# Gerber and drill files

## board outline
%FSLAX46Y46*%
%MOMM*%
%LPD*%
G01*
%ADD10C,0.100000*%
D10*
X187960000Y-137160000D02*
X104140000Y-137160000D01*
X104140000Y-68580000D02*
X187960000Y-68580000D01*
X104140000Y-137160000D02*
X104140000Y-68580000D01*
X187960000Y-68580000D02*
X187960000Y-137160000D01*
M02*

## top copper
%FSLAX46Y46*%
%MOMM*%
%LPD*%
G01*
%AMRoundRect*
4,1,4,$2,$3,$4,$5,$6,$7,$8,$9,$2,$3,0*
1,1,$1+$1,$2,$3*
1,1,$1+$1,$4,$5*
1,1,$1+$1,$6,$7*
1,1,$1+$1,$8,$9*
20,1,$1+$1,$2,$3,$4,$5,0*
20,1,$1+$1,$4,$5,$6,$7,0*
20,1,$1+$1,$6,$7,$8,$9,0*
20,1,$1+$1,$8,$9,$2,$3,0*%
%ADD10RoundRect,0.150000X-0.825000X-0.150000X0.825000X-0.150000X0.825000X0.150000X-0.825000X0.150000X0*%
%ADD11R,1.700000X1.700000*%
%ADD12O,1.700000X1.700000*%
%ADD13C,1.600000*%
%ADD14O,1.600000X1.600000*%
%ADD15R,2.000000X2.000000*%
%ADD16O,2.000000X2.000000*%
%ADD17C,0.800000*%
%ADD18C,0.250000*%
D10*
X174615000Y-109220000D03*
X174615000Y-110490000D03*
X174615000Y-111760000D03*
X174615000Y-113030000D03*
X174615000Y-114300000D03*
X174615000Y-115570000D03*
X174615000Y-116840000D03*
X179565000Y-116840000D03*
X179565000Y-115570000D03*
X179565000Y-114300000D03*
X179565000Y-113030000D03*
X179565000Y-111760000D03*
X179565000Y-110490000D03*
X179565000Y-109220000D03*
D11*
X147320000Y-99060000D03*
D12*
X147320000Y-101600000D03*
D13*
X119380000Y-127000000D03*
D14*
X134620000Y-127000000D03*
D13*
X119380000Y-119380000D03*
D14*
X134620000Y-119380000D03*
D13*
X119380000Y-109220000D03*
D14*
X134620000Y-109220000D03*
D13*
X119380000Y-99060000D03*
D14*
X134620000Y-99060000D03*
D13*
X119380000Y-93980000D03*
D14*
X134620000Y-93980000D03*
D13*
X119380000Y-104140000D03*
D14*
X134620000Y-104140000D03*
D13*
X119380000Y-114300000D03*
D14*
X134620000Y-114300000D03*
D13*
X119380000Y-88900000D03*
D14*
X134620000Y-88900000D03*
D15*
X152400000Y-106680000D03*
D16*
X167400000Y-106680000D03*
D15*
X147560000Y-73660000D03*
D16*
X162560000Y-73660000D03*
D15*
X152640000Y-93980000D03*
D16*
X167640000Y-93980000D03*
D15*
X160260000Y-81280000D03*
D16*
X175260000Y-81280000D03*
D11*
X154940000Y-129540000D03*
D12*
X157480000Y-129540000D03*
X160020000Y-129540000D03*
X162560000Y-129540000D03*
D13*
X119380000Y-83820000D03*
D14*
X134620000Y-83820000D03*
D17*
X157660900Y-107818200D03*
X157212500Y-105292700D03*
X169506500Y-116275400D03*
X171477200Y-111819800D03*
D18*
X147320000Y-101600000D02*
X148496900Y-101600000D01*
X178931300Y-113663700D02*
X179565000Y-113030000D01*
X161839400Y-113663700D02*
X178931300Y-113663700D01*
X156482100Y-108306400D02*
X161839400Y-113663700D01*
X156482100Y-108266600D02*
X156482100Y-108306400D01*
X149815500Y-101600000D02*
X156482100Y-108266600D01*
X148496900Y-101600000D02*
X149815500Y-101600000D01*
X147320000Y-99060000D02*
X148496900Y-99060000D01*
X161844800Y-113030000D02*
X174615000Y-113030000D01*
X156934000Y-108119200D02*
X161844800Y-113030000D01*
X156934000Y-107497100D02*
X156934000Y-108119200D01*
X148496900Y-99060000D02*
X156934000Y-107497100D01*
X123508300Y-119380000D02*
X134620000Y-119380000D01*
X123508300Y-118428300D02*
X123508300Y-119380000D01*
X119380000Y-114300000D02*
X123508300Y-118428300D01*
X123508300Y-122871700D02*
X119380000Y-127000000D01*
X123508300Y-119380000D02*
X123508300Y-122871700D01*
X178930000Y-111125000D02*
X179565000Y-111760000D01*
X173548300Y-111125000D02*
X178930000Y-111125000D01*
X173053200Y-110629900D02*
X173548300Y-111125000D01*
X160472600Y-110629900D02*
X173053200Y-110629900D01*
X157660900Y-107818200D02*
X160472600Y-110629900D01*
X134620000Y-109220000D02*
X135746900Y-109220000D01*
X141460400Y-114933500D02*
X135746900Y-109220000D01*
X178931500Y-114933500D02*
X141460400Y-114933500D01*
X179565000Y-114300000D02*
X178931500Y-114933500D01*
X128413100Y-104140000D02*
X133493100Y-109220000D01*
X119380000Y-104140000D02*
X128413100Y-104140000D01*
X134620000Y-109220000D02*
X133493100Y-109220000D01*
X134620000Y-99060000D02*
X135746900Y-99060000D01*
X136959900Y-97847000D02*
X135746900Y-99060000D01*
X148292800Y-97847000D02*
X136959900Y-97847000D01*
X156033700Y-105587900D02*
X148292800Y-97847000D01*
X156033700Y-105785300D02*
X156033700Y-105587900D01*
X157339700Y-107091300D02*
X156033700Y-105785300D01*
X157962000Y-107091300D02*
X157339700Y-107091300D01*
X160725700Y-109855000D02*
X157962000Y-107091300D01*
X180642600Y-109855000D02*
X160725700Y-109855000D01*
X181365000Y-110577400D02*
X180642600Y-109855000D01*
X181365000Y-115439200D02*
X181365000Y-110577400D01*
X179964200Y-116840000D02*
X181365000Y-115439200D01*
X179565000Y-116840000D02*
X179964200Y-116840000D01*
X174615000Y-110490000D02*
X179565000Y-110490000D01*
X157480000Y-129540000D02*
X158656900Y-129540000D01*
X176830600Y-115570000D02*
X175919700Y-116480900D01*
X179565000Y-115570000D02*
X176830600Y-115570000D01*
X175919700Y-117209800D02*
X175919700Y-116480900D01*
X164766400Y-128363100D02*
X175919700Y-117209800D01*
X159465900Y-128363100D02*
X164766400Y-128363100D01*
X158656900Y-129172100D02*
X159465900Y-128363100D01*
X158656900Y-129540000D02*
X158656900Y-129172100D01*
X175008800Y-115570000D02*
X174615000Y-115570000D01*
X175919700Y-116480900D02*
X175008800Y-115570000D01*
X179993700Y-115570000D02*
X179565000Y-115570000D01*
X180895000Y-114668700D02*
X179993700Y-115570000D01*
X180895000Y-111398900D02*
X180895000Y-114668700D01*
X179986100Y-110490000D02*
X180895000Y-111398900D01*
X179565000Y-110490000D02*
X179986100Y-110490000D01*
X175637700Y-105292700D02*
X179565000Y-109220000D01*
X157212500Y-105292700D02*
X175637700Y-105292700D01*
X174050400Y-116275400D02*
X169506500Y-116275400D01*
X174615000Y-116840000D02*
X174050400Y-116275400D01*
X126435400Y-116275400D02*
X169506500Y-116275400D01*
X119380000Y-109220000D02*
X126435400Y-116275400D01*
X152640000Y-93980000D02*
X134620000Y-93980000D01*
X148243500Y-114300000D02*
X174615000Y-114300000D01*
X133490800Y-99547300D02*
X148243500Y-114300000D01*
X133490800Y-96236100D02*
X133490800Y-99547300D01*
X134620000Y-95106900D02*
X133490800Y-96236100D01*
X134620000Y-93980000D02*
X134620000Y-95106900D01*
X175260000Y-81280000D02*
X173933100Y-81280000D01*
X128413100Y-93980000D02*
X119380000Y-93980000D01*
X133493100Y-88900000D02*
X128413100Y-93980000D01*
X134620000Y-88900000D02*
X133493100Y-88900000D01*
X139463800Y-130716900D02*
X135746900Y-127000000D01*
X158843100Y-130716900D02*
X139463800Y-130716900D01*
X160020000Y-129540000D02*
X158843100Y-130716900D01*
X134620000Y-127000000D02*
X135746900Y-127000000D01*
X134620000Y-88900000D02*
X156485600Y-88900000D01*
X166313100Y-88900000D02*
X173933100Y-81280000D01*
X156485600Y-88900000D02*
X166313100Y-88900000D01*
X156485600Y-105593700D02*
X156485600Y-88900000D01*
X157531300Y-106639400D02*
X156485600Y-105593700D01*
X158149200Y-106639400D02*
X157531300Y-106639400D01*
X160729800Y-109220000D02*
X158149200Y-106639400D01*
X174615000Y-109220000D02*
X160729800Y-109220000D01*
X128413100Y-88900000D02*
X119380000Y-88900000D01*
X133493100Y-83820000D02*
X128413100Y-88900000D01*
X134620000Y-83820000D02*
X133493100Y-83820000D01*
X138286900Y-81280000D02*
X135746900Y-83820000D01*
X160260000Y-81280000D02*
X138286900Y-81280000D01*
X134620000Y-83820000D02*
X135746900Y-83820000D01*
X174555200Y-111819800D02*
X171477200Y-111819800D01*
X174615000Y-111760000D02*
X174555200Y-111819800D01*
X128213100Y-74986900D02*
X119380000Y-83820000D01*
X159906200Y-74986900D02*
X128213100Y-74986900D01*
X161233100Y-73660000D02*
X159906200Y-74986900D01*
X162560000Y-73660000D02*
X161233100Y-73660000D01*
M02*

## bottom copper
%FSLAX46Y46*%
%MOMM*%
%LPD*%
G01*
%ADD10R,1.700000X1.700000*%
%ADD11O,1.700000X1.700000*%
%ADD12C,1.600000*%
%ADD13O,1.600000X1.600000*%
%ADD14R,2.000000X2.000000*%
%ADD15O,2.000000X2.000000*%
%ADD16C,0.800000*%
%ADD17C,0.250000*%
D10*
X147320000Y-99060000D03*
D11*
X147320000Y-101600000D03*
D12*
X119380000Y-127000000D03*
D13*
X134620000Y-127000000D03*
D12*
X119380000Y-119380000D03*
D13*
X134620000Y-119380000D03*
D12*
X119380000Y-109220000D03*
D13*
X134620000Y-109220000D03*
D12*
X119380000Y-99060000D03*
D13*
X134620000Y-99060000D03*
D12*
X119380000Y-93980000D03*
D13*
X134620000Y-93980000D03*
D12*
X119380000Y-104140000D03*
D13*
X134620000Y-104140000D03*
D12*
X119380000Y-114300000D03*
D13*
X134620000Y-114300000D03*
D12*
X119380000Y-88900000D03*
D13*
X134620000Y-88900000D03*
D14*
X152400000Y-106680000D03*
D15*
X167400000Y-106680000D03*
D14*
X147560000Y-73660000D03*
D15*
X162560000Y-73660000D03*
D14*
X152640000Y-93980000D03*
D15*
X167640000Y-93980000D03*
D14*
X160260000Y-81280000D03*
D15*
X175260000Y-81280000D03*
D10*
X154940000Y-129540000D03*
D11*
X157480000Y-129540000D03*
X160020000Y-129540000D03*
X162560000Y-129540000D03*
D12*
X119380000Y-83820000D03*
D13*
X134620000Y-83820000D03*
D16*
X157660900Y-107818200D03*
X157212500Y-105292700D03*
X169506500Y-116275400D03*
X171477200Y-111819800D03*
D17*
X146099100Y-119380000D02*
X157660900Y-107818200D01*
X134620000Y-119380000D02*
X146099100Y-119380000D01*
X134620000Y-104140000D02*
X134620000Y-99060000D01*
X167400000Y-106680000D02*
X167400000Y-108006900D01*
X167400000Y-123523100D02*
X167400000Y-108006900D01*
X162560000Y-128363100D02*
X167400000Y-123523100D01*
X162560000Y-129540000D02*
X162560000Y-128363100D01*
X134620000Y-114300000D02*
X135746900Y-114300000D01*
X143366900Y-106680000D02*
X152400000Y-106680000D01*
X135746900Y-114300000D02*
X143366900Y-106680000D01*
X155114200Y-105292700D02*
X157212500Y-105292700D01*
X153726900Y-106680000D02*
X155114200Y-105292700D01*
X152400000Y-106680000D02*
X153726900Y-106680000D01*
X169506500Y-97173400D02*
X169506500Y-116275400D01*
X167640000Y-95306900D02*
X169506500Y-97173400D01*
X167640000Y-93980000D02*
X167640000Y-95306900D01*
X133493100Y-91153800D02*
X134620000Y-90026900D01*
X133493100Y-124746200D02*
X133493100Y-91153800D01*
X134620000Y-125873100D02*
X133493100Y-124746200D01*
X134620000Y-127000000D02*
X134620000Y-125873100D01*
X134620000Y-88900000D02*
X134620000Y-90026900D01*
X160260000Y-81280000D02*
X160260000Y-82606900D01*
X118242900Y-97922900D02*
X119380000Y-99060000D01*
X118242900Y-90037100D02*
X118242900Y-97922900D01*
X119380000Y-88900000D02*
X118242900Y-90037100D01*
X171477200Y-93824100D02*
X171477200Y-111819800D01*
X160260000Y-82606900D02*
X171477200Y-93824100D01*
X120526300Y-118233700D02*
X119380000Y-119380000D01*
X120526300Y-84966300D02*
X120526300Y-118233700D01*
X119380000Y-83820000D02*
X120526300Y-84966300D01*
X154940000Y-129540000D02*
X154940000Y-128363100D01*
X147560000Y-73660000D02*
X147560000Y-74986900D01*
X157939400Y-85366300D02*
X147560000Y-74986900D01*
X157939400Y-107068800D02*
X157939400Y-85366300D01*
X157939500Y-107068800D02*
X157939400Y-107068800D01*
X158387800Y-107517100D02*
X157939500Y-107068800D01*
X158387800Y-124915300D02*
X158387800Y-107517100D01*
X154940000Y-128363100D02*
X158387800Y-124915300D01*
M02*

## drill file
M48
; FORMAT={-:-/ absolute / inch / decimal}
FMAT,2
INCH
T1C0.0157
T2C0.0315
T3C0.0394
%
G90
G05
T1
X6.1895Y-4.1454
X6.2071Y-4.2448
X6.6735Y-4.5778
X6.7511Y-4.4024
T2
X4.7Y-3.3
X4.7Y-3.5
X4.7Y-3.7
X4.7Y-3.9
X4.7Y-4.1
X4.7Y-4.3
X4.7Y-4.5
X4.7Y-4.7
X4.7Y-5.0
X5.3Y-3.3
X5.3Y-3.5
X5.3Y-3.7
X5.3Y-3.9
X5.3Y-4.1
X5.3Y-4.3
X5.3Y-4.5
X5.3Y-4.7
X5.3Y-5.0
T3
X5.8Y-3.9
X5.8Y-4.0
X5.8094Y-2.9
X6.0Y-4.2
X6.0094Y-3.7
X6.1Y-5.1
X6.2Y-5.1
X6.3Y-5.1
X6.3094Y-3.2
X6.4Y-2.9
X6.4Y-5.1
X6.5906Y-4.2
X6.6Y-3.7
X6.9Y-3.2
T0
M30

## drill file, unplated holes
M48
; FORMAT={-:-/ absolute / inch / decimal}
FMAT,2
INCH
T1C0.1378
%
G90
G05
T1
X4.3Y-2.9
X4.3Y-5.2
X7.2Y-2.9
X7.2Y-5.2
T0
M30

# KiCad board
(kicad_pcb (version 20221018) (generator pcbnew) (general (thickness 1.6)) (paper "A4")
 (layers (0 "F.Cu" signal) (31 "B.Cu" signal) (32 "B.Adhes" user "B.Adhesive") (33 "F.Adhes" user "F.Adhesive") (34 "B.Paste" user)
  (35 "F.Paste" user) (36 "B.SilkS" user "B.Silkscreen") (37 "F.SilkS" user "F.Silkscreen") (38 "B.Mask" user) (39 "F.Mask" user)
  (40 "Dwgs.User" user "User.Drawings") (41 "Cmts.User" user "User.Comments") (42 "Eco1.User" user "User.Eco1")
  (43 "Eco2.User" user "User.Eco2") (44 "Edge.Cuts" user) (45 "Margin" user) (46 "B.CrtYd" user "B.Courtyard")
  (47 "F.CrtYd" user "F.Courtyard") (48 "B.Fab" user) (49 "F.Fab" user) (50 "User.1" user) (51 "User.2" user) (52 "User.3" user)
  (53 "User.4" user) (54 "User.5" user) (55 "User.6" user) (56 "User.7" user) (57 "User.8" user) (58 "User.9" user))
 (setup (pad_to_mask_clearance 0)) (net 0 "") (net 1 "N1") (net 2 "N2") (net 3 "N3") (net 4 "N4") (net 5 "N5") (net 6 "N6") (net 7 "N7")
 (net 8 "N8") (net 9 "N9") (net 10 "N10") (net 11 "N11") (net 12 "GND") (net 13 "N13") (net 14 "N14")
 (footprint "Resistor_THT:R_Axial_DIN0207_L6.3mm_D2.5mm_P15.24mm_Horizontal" (layer "F.Cu") (at 119.38 127)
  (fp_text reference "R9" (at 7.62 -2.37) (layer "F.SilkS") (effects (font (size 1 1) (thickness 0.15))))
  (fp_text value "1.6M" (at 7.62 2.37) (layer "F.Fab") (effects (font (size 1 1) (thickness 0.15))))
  (pad "1" thru_hole circle (at 0 0) (size 1.6 1.6) (drill 0.8) (layers "*.Cu" "*.Mask") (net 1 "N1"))
  (pad "2" thru_hole oval (at 15.24 0) (size 1.6 1.6) (drill 0.8) (layers "*.Cu" "*.Mask") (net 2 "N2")))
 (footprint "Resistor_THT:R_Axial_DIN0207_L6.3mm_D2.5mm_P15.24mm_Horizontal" (layer "F.Cu") (at 119.38 119.38)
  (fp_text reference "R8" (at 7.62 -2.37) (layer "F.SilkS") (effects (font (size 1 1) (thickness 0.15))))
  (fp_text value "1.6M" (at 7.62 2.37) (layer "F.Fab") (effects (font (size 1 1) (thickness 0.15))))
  (pad "1" thru_hole circle (at 0 0) (size 1.6 1.6) (drill 0.8) (layers "*.Cu" "*.Mask") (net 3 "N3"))
  (pad "2" thru_hole oval (at 15.24 0) (size 1.6 1.6) (drill 0.8) (layers "*.Cu" "*.Mask") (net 1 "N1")))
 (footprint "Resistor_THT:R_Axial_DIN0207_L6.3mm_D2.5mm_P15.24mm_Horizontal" (layer "F.Cu") (at 119.38 109.22)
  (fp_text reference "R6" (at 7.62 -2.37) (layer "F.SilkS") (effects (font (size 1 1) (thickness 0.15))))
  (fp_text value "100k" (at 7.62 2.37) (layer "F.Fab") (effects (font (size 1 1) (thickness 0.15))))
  (pad "1" thru_hole circle (at 0 0) (size 1.6 1.6) (drill 0.8) (layers "*.Cu" "*.Mask") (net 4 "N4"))
  (pad "2" thru_hole oval (at 15.24 0) (size 1.6 1.6) (drill 0.8) (layers "*.Cu" "*.Mask") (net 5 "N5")))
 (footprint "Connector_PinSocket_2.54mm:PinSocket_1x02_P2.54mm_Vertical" (layer "F.Cu") (at 147.32 99.06)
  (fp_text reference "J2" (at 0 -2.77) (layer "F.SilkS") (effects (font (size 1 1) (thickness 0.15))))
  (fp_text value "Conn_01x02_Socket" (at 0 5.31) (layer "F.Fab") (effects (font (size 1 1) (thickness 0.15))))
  (pad "1" thru_hole rect (at 0 0) (size 1.7 1.7) (drill 1) (layers "*.Cu" "*.Mask") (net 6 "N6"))
  (pad "2" thru_hole oval (at 0 2.54) (size 1.7 1.7) (drill 1) (layers "*.Cu" "*.Mask") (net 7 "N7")))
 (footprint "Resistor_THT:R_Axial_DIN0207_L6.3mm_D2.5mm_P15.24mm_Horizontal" (layer "F.Cu") (at 119.38 99.06)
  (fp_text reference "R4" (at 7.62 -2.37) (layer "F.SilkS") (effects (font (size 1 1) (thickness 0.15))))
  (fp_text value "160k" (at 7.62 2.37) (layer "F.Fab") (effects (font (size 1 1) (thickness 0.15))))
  (pad "1" thru_hole circle (at 0 0) (size 1.6 1.6) (drill 0.8) (layers "*.Cu" "*.Mask") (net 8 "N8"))
  (pad "2" thru_hole oval (at 15.24 0) (size 1.6 1.6) (drill 0.8) (layers "*.Cu" "*.Mask") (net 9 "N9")))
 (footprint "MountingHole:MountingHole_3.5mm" (layer "F.Cu") (at 109.22 132.08)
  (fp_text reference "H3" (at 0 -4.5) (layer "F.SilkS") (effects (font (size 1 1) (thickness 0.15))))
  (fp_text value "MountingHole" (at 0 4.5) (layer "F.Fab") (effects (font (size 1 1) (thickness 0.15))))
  (pad "" np_thru_hole circle (at 0 0) (size 3.5 3.5) (drill 3.5) (layers "*.Cu" "*.Mask")))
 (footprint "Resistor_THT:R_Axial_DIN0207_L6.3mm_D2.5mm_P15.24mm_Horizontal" (layer "F.Cu") (at 119.38 93.98)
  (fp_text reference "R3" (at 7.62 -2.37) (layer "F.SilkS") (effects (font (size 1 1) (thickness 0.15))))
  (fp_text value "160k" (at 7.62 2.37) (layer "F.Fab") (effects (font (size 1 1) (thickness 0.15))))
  (pad "1" thru_hole circle (at 0 0) (size 1.6 1.6) (drill 0.8) (layers "*.Cu" "*.Mask") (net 2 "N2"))
  (pad "2" thru_hole oval (at 15.24 0) (size 1.6 1.6) (drill 0.8) (layers "*.Cu" "*.Mask") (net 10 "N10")))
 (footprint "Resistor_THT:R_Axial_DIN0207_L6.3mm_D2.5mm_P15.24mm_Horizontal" (layer "F.Cu") (at 119.38 104.14)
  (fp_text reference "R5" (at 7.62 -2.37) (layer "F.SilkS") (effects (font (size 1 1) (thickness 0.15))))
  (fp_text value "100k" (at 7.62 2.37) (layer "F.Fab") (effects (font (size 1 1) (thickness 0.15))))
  (pad "1" thru_hole circle (at 0 0) (size 1.6 1.6) (drill 0.8) (layers "*.Cu" "*.Mask") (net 5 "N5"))
  (pad "2" thru_hole oval (at 15.24 0) (size 1.6 1.6) (drill 0.8) (layers "*.Cu" "*.Mask") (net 9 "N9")))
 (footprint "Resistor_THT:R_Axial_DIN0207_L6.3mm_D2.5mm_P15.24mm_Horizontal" (layer "F.Cu") (at 119.38 114.3)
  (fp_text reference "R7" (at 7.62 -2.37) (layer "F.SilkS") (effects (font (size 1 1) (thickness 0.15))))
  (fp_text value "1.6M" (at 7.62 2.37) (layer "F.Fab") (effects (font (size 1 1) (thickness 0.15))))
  (pad "1" thru_hole circle (at 0 0) (size 1.6 1.6) (drill 0.8) (layers "*.Cu" "*.Mask") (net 1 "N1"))
  (pad "2" thru_hole oval (at 15.24 0) (size 1.6 1.6) (drill 0.8) (layers "*.Cu" "*.Mask") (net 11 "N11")))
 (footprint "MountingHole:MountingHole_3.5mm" (layer "F.Cu") (at 109.22 73.66)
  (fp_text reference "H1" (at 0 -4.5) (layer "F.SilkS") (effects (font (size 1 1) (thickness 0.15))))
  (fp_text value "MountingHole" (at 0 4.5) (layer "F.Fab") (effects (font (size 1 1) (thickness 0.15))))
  (pad "" np_thru_hole circle (at 0 0) (size 3.5 3.5) (drill 3.5) (layers "*.Cu" "*.Mask")))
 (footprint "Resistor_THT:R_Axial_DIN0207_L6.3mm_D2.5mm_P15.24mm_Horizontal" (layer "F.Cu") (at 119.38 88.9)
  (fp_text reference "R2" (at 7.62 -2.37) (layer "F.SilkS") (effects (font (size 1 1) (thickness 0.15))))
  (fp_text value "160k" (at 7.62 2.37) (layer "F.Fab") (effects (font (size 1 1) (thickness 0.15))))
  (pad "1" thru_hole circle (at 0 0) (size 1.6 1.6) (drill 0.8) (layers "*.Cu" "*.Mask") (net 8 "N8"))
  (pad "2" thru_hole oval (at 15.24 0) (size 1.6 1.6) (drill 0.8) (layers "*.Cu" "*.Mask") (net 2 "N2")))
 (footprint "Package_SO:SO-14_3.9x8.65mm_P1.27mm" (layer "F.Cu") (at 177.09 113.03)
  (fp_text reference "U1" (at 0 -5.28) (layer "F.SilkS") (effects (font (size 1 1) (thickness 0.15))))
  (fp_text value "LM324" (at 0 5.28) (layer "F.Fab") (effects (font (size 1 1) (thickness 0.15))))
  (pad "1" smd roundrect (at -2.475 -3.81) (size 1.95 0.6) (layers "F.Cu" "F.Paste" "F.Mask") (roundrect_rratio 0.25) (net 2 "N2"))
  (pad "2" smd roundrect (at -2.475 -2.54) (size 1.95 0.6) (layers "F.Cu" "F.Paste" "F.Mask") (roundrect_rratio 0.25) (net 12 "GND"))
  (pad "3" smd roundrect (at -2.475 -1.27) (size 1.95 0.6) (layers "F.Cu" "F.Paste" "F.Mask") (roundrect_rratio 0.25) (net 8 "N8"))
  (pad "4" smd roundrect (at -2.475 0) (size 1.95 0.6) (layers "F.Cu" "F.Paste" "F.Mask") (roundrect_rratio 0.25) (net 6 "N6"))
  (pad "5" smd roundrect (at -2.475 1.27) (size 1.95 0.6) (layers "F.Cu" "F.Paste" "F.Mask") (roundrect_rratio 0.25) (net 10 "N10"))
  (pad "6" smd roundrect (at -2.475 2.54) (size 1.95 0.6) (layers "F.Cu" "F.Paste" "F.Mask") (roundrect_rratio 0.25) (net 12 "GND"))
  (pad "7" smd roundrect (at -2.475 3.81) (size 1.95 0.6) (layers "F.Cu" "F.Paste" "F.Mask") (roundrect_rratio 0.25) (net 4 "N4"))
  (pad "8" smd roundrect (at 2.475 3.81) (size 1.95 0.6) (layers "F.Cu" "F.Paste" "F.Mask") (roundrect_rratio 0.25) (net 9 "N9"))
  (pad "9" smd roundrect (at 2.475 2.54) (size 1.95 0.6) (layers "F.Cu" "F.Paste" "F.Mask") (roundrect_rratio 0.25) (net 12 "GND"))
  (pad "10" smd roundrect (at 2.475 1.27) (size 1.95 0.6) (layers "F.Cu" "F.Paste" "F.Mask") (roundrect_rratio 0.25) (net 5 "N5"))
  (pad "11" smd roundrect (at 2.475 0) (size 1.95 0.6) (layers "F.Cu" "F.Paste" "F.Mask") (roundrect_rratio 0.25) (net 7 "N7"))
  (pad "12" smd roundrect (at 2.475 -1.27) (size 1.95 0.6) (layers "F.Cu" "F.Paste" "F.Mask") (roundrect_rratio 0.25) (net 1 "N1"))
  (pad "13" smd roundrect (at 2.475 -2.54) (size 1.95 0.6) (layers "F.Cu" "F.Paste" "F.Mask") (roundrect_rratio 0.25) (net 12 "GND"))
  (pad "14" smd roundrect (at 2.475 -3.81) (size 1.95 0.6) (layers "F.Cu" "F.Paste" "F.Mask") (roundrect_rratio 0.25) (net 11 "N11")))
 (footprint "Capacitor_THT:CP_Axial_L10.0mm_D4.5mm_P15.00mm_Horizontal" (layer "F.Cu") (at 152.4 106.68)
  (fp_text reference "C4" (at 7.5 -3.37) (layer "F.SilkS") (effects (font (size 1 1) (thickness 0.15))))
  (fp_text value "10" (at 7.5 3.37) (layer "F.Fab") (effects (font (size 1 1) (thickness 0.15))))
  (pad "1" thru_hole rect (at 0 0) (size 2 2) (drill 1) (layers "*.Cu" "*.Mask") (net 11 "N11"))
  (pad "2" thru_hole oval (at 15 0) (size 2 2) (drill 1) (layers "*.Cu" "*.Mask") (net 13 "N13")))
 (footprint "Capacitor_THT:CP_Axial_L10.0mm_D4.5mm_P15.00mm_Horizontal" (layer "F.Cu") (at 147.56 73.66)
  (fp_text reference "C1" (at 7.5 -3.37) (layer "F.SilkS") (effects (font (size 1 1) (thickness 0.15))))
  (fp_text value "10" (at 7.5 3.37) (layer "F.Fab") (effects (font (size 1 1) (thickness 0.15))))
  (pad "1" thru_hole rect (at 0 0) (size 2 2) (drill 1) (layers "*.Cu" "*.Mask") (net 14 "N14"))
  (pad "2" thru_hole oval (at 15 0) (size 2 2) (drill 1) (layers "*.Cu" "*.Mask") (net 3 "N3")))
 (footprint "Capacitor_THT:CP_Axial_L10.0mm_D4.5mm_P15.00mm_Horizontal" (layer "F.Cu") (at 152.64 93.98)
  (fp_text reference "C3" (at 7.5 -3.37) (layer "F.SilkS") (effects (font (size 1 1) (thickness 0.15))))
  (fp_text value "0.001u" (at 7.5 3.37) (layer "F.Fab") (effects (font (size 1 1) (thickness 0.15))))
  (pad "1" thru_hole rect (at 0 0) (size 2 2) (drill 1) (layers "*.Cu" "*.Mask") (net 10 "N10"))
  (pad "2" thru_hole oval (at 15 0) (size 2 2) (drill 1) (layers "*.Cu" "*.Mask") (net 4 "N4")))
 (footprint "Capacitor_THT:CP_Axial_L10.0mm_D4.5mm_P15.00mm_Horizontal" (layer "F.Cu") (at 160.26 81.28)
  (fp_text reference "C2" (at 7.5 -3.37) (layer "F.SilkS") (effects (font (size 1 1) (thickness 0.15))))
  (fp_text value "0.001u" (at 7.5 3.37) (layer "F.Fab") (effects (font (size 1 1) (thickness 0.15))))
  (pad "1" thru_hole rect (at 0 0) (size 2 2) (drill 1) (layers "*.Cu" "*.Mask") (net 8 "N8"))
  (pad "2" thru_hole oval (at 15 0) (size 2 2) (drill 1) (layers "*.Cu" "*.Mask") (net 2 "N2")))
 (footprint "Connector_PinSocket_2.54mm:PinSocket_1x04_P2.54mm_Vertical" (layer "F.Cu") (at 154.94 129.54 90)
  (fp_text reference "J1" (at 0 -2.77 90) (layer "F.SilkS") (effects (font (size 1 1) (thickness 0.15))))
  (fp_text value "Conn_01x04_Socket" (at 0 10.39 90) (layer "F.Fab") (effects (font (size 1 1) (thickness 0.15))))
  (pad "1" thru_hole rect (at 0 0 90) (size 1.7 1.7) (drill 1) (layers "*.Cu" "*.Mask") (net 14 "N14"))
  (pad "2" thru_hole oval (at 0 2.54 90) (size 1.7 1.7) (drill 1) (layers "*.Cu" "*.Mask") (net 12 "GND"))
  (pad "3" thru_hole oval (at 0 5.08 90) (size 1.7 1.7) (drill 1) (layers "*.Cu" "*.Mask") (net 2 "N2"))
  (pad "4" thru_hole oval (at 0 7.62 90) (size 1.7 1.7) (drill 1) (layers "*.Cu" "*.Mask") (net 13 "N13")))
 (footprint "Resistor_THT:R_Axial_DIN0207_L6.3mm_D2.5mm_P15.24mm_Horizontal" (layer "F.Cu") (at 119.38 83.82)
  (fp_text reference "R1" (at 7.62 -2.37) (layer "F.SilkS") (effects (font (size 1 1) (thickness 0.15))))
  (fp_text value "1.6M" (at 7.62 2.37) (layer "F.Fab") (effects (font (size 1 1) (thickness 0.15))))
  (pad "1" thru_hole circle (at 0 0) (size 1.6 1.6) (drill 0.8) (layers "*.Cu" "*.Mask") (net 3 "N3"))
  (pad "2" thru_hole oval (at 15.24 0) (size 1.6 1.6) (drill 0.8) (layers "*.Cu" "*.Mask") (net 8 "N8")))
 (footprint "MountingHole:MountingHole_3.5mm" (layer "F.Cu") (at 182.88 132.08)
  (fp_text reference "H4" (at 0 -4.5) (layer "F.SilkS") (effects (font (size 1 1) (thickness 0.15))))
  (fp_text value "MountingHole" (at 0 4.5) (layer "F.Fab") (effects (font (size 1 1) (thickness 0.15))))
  (pad "" np_thru_hole circle (at 0 0) (size 3.5 3.5) (drill 3.5) (layers "*.Cu" "*.Mask")))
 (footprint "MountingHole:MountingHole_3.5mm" (layer "F.Cu") (at 182.88 73.66)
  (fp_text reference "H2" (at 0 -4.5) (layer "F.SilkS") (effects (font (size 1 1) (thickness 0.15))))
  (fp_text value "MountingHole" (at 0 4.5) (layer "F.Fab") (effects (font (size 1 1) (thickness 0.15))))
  (pad "" np_thru_hole circle (at 0 0) (size 3.5 3.5) (drill 3.5) (layers "*.Cu" "*.Mask")))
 (gr_line (start 187.96 137.16) (end 104.14 137.16) (stroke (width 0.1) (type default)) (layer "Edge.Cuts"))
 (gr_line (start 104.14 68.58) (end 187.96 68.58) (stroke (width 0.1) (type default)) (layer "Edge.Cuts"))
 (gr_line (start 104.14 137.16) (end 104.14 68.58) (stroke (width 0.1) (type default)) (layer "Edge.Cuts"))
 (gr_line (start 187.96 68.58) (end 187.96 137.16) (stroke (width 0.1) (type default)) (layer "Edge.Cuts"))
 (segment (start 157.9395 107.0688) (end 157.9394 107.0688) (width 0.25) (layer "B.Cu") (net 14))
 (segment (start 154.94 128.3631) (end 158.3878 124.9153) (width 0.25) (layer "B.Cu") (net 14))
 (segment (start 154.94 129.54) (end 154.94 128.3631) (width 0.25) (layer "B.Cu") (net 14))
 (segment (start 157.9394 85.3663) (end 147.56 74.9869) (width 0.25) (layer "B.Cu") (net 14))
 (segment (start 158.3878 124.9153) (end 158.3878 107.5171) (width 0.25) (layer "B.Cu") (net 14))
 (segment (start 157.9394 107.0688) (end 157.9394 85.3663) (width 0.25) (layer "B.Cu") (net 14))
 (segment (start 147.56 73.66) (end 147.56 74.9869) (width 0.25) (layer "B.Cu") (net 14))
 (segment (start 158.3878 107.5171) (end 157.9395 107.0688) (width 0.25) (layer "B.Cu") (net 14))
 (segment (start 162.56 73.66) (end 161.2331 73.66) (width 0.25) (layer "F.Cu") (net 3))
 (segment (start 128.2131 74.9869) (end 119.38 83.82) (width 0.25) (layer "F.Cu") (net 3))
 (segment (start 159.9062 74.9869) (end 128.2131 74.9869) (width 0.25) (layer "F.Cu") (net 3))
 (segment (start 161.2331 73.66) (end 159.9062 74.9869) (width 0.25) (layer "F.Cu") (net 3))
 (segment (start 119.38 83.82) (end 120.5263 84.9663) (width 0.25) (layer "B.Cu") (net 3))
 (segment (start 120.5263 118.2337) (end 119.38 119.38) (width 0.25) (layer "B.Cu") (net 3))
 (segment (start 120.5263 84.9663) (end 120.5263 118.2337) (width 0.25) (layer "B.Cu") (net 3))
 (segment (start 160.26 81.28) (end 138.2869 81.28) (width 0.25) (layer "F.Cu") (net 8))
 (segment (start 138.2869 81.28) (end 135.7469 83.82) (width 0.25) (layer "F.Cu") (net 8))
 (segment (start 128.4131 88.9) (end 119.38 88.9) (width 0.25) (layer "F.Cu") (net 8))
 (segment (start 133.4931 83.82) (end 128.4131 88.9) (width 0.25) (layer "F.Cu") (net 8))
 (segment (start 134.62 83.82) (end 135.7469 83.82) (width 0.25) (layer "F.Cu") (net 8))
 (segment (start 134.62 83.82) (end 133.4931 83.82) (width 0.25) (layer "F.Cu") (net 8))
 (segment (start 174.5552 111.8198) (end 171.4772 111.8198) (width 0.25) (layer "F.Cu") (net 8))
 (segment (start 174.615 111.76) (end 174.5552 111.8198) (width 0.25) (layer "F.Cu") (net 8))
 (via (at 171.4772 111.8198) (size 0.8) (drill 0.4) (layers "F.Cu" "B.Cu") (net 8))
 (segment (start 160.26 82.6069) (end 171.4772 93.8241) (width 0.25) (layer "B.Cu") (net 8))
 (segment (start 118.2429 97.9229) (end 119.38 99.06) (width 0.25) (layer "B.Cu") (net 8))
 (segment (start 119.38 88.9) (end 118.2429 90.0371) (width 0.25) (layer "B.Cu") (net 8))
 (segment (start 160.26 81.28) (end 160.26 82.6069) (width 0.25) (layer "B.Cu") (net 8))
 (segment (start 171.4772 93.8241) (end 171.4772 111.8198) (width 0.25) (layer "B.Cu") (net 8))
 (segment (start 118.2429 90.0371) (end 118.2429 97.9229) (width 0.25) (layer "B.Cu") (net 8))
 (segment (start 158.1492 106.6394) (end 157.5313 106.6394) (width 0.25) (layer "F.Cu") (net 2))
 (segment (start 134.62 127) (end 135.7469 127) (width 0.25) (layer "F.Cu") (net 2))
 (segment (start 156.4856 88.9) (end 166.3131 88.9) (width 0.25) (layer "F.Cu") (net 2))
 (segment (start 174.615 109.22) (end 160.7298 109.22) (width 0.25) (layer "F.Cu") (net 2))
 (segment (start 134.62 88.9) (end 133.4931 88.9) (width 0.25) (layer "F.Cu") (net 2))
 (segment (start 156.4856 105.5937) (end 156.4856 88.9) (width 0.25) (layer "F.Cu") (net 2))
 (segment (start 157.5313 106.6394) (end 156.4856 105.5937) (width 0.25) (layer "F.Cu") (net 2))
 (segment (start 133.4931 88.9) (end 128.4131 93.98) (width 0.25) (layer "F.Cu") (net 2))
 (segment (start 128.4131 93.98) (end 119.38 93.98) (width 0.25) (layer "F.Cu") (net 2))
 (segment (start 134.62 88.9) (end 156.4856 88.9) (width 0.25) (layer "F.Cu") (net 2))
 (segment (start 175.26 81.28) (end 173.9331 81.28) (width 0.25) (layer "F.Cu") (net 2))
 (segment (start 139.4638 130.7169) (end 135.7469 127) (width 0.25) (layer "F.Cu") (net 2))
 (segment (start 158.8431 130.7169) (end 139.4638 130.7169) (width 0.25) (layer "F.Cu") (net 2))
 (segment (start 160.7298 109.22) (end 158.1492 106.6394) (width 0.25) (layer "F.Cu") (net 2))
 (segment (start 166.3131 88.9) (end 173.9331 81.28) (width 0.25) (layer "F.Cu") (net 2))
 (segment (start 160.02 129.54) (end 158.8431 130.7169) (width 0.25) (layer "F.Cu") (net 2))
 (segment (start 134.62 127) (end 134.62 125.8731) (width 0.25) (layer "B.Cu") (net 2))
 (segment (start 134.62 125.8731) (end 133.4931 124.7462) (width 0.25) (layer "B.Cu") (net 2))
 (segment (start 133.4931 91.1538) (end 134.62 90.0269) (width 0.25) (layer "B.Cu") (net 2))
 (segment (start 133.4931 124.7462) (end 133.4931 91.1538) (width 0.25) (layer "B.Cu") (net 2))
 (segment (start 134.62 88.9) (end 134.62 90.0269) (width 0.25) (layer "B.Cu") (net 2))
 (segment (start 148.2435 114.3) (end 174.615 114.3) (width 0.25) (layer "F.Cu") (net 10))
 (segment (start 133.4908 96.2361) (end 133.4908 99.5473) (width 0.25) (layer "F.Cu") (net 10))
 (segment (start 133.4908 99.5473) (end 148.2435 114.3) (width 0.25) (layer "F.Cu") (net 10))
 (segment (start 134.62 93.98) (end 134.62 95.1069) (width 0.25) (layer "F.Cu") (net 10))
 (segment (start 152.64 93.98) (end 134.62 93.98) (width 0.25) (layer "F.Cu") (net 10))
 (segment (start 134.62 95.1069) (end 133.4908 96.2361) (width 0.25) (layer "F.Cu") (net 10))
 (segment (start 119.38 109.22) (end 126.4354 116.2754) (width 0.25) (layer "F.Cu") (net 4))
 (segment (start 174.615 116.84) (end 174.0504 116.2754) (width 0.25) (layer "F.Cu") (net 4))
 (segment (start 174.0504 116.2754) (end 169.5065 116.2754) (width 0.25) (layer "F.Cu") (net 4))
 (segment (start 126.4354 116.2754) (end 169.5065 116.2754) (width 0.25) (layer "F.Cu") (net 4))
 (via (at 169.5065 116.2754) (size 0.8) (drill 0.4) (layers "F.Cu" "B.Cu") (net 4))
 (segment (start 167.64 93.98) (end 167.64 95.3069) (width 0.25) (layer "B.Cu") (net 4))
 (segment (start 167.64 95.3069) (end 169.5065 97.1734) (width 0.25) (layer "B.Cu") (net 4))
 (segment (start 169.5065 97.1734) (end 169.5065 116.2754) (width 0.25) (layer "B.Cu") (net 4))
 (segment (start 175.6377 105.2927) (end 179.565 109.22) (width 0.25) (layer "F.Cu") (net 11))
 (segment (start 157.2125 105.2927) (end 175.6377 105.2927) (width 0.25) (layer "F.Cu") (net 11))
 (via (at 157.2125 105.2927) (size 0.8) (drill 0.4) (layers "F.Cu" "B.Cu") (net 11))
 (segment (start 134.62 114.3) (end 135.7469 114.3) (width 0.25) (layer "B.Cu") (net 11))
 (segment (start 152.4 106.68) (end 153.7269 106.68) (width 0.25) (layer "B.Cu") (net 11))
 (segment (start 143.3669 106.68) (end 152.4 106.68) (width 0.25) (layer "B.Cu") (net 11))
 (segment (start 153.7269 106.68) (end 155.1142 105.2927) (width 0.25) (layer "B.Cu") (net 11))
 (segment (start 135.7469 114.3) (end 143.3669 106.68) (width 0.25) (layer "B.Cu") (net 11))
 (segment (start 155.1142 105.2927) (end 157.2125 105.2927) (width 0.25) (layer "B.Cu") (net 11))
 (segment (start 167.4 123.5231) (end 167.4 108.0069) (width 0.25) (layer "B.Cu") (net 13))
 (segment (start 167.4 106.68) (end 167.4 108.0069) (width 0.25) (layer "B.Cu") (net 13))
 (segment (start 162.56 128.3631) (end 167.4 123.5231) (width 0.25) (layer "B.Cu") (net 13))
 (segment (start 162.56 129.54) (end 162.56 128.3631) (width 0.25) (layer "B.Cu") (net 13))
 (segment (start 179.565 110.49) (end 179.9861 110.49) (width 0.25) (layer "F.Cu") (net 12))
 (segment (start 157.48 129.54) (end 158.6569 129.54) (width 0.25) (layer "F.Cu") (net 12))
 (segment (start 164.7664 128.3631) (end 175.9197 117.2098) (width 0.25) (layer "F.Cu") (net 12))
 (segment (start 180.895 114.6687) (end 179.9937 115.57) (width 0.25) (layer "F.Cu") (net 12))
 (segment (start 158.6569 129.54) (end 158.6569 129.1721) (width 0.25) (layer "F.Cu") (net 12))
 (segment (start 176.8306 115.57) (end 175.9197 116.4809) (width 0.25) (layer "F.Cu") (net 12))
 (segment (start 179.565 115.57) (end 176.8306 115.57) (width 0.25) (layer "F.Cu") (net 12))
 (segment (start 159.4659 128.3631) (end 164.7664 128.3631) (width 0.25) (layer "F.Cu") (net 12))
 (segment (start 175.0088 115.57) (end 174.615 115.57) (width 0.25) (layer "F.Cu") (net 12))
 (segment (start 158.6569 129.1721) (end 159.4659 128.3631) (width 0.25) (layer "F.Cu") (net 12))
 (segment (start 175.9197 116.4809) (end 175.0088 115.57) (width 0.25) (layer "F.Cu") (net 12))
 (segment (start 179.9861 110.49) (end 180.895 111.3989) (width 0.25) (layer "F.Cu") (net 12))
 (segment (start 180.895 111.3989) (end 180.895 114.6687) (width 0.25) (layer "F.Cu") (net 12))
 (segment (start 179.9937 115.57) (end 179.565 115.57) (width 0.25) (layer "F.Cu") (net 12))
 (segment (start 174.615 110.49) (end 179.565 110.49) (width 0.25) (layer "F.Cu") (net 12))
 (segment (start 175.9197 117.2098) (end 175.9197 116.4809) (width 0.25) (layer "F.Cu") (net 12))
 (segment (start 160.7257 109.855) (end 157.962 107.0913) (width 0.25) (layer "F.Cu") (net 9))
 (segment (start 181.365 110.5774) (end 180.6426 109.855) (width 0.25) (layer "F.Cu") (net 9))
 (segment (start 156.0337 105.7853) (end 156.0337 105.5879) (width 0.25) (layer "F.Cu") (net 9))
 (segment (start 157.3397 107.0913) (end 156.0337 105.7853) (width 0.25) (layer "F.Cu") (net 9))
 (segment (start 148.2928 97.847) (end 136.9599 97.847) (width 0.25) (layer "F.Cu") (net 9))
 (segment (start 134.62 99.06) (end 135.7469 99.06) (width 0.25) (layer "F.Cu") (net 9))
 (segment (start 156.0337 105.5879) (end 148.2928 97.847) (width 0.25) (layer "F.Cu") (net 9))
 (segment (start 136.9599 97.847) (end 135.7469 99.06) (width 0.25) (layer "F.Cu") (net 9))
 (segment (start 181.365 115.4392) (end 181.365 110.5774) (width 0.25) (layer "F.Cu") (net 9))
 (segment (start 179.9642 116.84) (end 181.365 115.4392) (width 0.25) (layer "F.Cu") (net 9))
 (segment (start 157.962 107.0913) (end 157.3397 107.0913) (width 0.25) (layer "F.Cu") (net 9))
 (segment (start 180.6426 109.855) (end 160.7257 109.855) (width 0.25) (layer "F.Cu") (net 9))
 (segment (start 179.565 116.84) (end 179.9642 116.84) (width 0.25) (layer "F.Cu") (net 9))
 (segment (start 134.62 104.14) (end 134.62 99.06) (width 0.25) (layer "B.Cu") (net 9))
 (segment (start 179.565 114.3) (end 178.9315 114.9335) (width 0.25) (layer "F.Cu") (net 5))
 (segment (start 128.4131 104.14) (end 133.4931 109.22) (width 0.25) (layer "F.Cu") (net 5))
 (segment (start 134.62 109.22) (end 135.7469 109.22) (width 0.25) (layer "F.Cu") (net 5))
 (segment (start 119.38 104.14) (end 128.4131 104.14) (width 0.25) (layer "F.Cu") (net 5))
 (segment (start 178.9315 114.9335) (end 141.4604 114.9335) (width 0.25) (layer "F.Cu") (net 5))
 (segment (start 141.4604 114.9335) (end 135.7469 109.22) (width 0.25) (layer "F.Cu") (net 5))
 (segment (start 134.62 109.22) (end 133.4931 109.22) (width 0.25) (layer "F.Cu") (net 5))
 (segment (start 123.5083 119.38) (end 123.5083 122.8717) (width 0.25) (layer "F.Cu") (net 1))
 (segment (start 157.6609 107.8182) (end 160.4726 110.6299) (width 0.25) (layer "F.Cu") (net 1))
 (segment (start 173.0532 110.6299) (end 173.5483 111.125) (width 0.25) (layer "F.Cu") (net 1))
 (segment (start 119.38 114.3) (end 123.5083 118.4283) (width 0.25) (layer "F.Cu") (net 1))
 (segment (start 178.93 111.125) (end 179.565 111.76) (width 0.25) (layer "F.Cu") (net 1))
 (segment (start 123.5083 122.8717) (end 119.38 127) (width 0.25) (layer "F.Cu") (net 1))
 (segment (start 123.5083 118.4283) (end 123.5083 119.38) (width 0.25) (layer "F.Cu") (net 1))
 (segment (start 173.5483 111.125) (end 178.93 111.125) (width 0.25) (layer "F.Cu") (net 1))
 (segment (start 123.5083 119.38) (end 134.62 119.38) (width 0.25) (layer "F.Cu") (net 1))
 (segment (start 160.4726 110.6299) (end 173.0532 110.6299) (width 0.25) (layer "F.Cu") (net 1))
 (via (at 157.6609 107.8182) (size 0.8) (drill 0.4) (layers "F.Cu" "B.Cu") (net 1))
 (segment (start 134.62 119.38) (end 146.0991 119.38) (width 0.25) (layer "B.Cu") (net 1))
 (segment (start 146.0991 119.38) (end 157.6609 107.8182) (width 0.25) (layer "B.Cu") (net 1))
 (segment (start 161.8448 113.03) (end 174.615 113.03) (width 0.25) (layer "F.Cu") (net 6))
 (segment (start 148.4969 99.06) (end 156.934 107.4971) (width 0.25) (layer "F.Cu") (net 6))
 (segment (start 147.32 99.06) (end 148.4969 99.06) (width 0.25) (layer "F.Cu") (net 6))
 (segment (start 156.934 108.1192) (end 161.8448 113.03) (width 0.25) (layer "F.Cu") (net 6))
 (segment (start 156.934 107.4971) (end 156.934 108.1192) (width 0.25) (layer "F.Cu") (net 6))
 (segment (start 161.8394 113.6637) (end 178.9313 113.6637) (width 0.25) (layer "F.Cu") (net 7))
 (segment (start 178.9313 113.6637) (end 179.565 113.03) (width 0.25) (layer "F.Cu") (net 7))
 (segment (start 149.8155 101.6) (end 156.4821 108.2666) (width 0.25) (layer "F.Cu") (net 7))
 (segment (start 156.4821 108.3064) (end 161.8394 113.6637) (width 0.25) (layer "F.Cu") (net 7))
 (segment (start 156.4821 108.2666) (end 156.4821 108.3064) (width 0.25) (layer "F.Cu") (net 7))
 (segment (start 148.4969 101.6) (end 149.8155 101.6) (width 0.25) (layer "F.Cu") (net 7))
 (segment (start 147.32 101.6) (end 148.4969 101.6) (width 0.25) (layer "F.Cu") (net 7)))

